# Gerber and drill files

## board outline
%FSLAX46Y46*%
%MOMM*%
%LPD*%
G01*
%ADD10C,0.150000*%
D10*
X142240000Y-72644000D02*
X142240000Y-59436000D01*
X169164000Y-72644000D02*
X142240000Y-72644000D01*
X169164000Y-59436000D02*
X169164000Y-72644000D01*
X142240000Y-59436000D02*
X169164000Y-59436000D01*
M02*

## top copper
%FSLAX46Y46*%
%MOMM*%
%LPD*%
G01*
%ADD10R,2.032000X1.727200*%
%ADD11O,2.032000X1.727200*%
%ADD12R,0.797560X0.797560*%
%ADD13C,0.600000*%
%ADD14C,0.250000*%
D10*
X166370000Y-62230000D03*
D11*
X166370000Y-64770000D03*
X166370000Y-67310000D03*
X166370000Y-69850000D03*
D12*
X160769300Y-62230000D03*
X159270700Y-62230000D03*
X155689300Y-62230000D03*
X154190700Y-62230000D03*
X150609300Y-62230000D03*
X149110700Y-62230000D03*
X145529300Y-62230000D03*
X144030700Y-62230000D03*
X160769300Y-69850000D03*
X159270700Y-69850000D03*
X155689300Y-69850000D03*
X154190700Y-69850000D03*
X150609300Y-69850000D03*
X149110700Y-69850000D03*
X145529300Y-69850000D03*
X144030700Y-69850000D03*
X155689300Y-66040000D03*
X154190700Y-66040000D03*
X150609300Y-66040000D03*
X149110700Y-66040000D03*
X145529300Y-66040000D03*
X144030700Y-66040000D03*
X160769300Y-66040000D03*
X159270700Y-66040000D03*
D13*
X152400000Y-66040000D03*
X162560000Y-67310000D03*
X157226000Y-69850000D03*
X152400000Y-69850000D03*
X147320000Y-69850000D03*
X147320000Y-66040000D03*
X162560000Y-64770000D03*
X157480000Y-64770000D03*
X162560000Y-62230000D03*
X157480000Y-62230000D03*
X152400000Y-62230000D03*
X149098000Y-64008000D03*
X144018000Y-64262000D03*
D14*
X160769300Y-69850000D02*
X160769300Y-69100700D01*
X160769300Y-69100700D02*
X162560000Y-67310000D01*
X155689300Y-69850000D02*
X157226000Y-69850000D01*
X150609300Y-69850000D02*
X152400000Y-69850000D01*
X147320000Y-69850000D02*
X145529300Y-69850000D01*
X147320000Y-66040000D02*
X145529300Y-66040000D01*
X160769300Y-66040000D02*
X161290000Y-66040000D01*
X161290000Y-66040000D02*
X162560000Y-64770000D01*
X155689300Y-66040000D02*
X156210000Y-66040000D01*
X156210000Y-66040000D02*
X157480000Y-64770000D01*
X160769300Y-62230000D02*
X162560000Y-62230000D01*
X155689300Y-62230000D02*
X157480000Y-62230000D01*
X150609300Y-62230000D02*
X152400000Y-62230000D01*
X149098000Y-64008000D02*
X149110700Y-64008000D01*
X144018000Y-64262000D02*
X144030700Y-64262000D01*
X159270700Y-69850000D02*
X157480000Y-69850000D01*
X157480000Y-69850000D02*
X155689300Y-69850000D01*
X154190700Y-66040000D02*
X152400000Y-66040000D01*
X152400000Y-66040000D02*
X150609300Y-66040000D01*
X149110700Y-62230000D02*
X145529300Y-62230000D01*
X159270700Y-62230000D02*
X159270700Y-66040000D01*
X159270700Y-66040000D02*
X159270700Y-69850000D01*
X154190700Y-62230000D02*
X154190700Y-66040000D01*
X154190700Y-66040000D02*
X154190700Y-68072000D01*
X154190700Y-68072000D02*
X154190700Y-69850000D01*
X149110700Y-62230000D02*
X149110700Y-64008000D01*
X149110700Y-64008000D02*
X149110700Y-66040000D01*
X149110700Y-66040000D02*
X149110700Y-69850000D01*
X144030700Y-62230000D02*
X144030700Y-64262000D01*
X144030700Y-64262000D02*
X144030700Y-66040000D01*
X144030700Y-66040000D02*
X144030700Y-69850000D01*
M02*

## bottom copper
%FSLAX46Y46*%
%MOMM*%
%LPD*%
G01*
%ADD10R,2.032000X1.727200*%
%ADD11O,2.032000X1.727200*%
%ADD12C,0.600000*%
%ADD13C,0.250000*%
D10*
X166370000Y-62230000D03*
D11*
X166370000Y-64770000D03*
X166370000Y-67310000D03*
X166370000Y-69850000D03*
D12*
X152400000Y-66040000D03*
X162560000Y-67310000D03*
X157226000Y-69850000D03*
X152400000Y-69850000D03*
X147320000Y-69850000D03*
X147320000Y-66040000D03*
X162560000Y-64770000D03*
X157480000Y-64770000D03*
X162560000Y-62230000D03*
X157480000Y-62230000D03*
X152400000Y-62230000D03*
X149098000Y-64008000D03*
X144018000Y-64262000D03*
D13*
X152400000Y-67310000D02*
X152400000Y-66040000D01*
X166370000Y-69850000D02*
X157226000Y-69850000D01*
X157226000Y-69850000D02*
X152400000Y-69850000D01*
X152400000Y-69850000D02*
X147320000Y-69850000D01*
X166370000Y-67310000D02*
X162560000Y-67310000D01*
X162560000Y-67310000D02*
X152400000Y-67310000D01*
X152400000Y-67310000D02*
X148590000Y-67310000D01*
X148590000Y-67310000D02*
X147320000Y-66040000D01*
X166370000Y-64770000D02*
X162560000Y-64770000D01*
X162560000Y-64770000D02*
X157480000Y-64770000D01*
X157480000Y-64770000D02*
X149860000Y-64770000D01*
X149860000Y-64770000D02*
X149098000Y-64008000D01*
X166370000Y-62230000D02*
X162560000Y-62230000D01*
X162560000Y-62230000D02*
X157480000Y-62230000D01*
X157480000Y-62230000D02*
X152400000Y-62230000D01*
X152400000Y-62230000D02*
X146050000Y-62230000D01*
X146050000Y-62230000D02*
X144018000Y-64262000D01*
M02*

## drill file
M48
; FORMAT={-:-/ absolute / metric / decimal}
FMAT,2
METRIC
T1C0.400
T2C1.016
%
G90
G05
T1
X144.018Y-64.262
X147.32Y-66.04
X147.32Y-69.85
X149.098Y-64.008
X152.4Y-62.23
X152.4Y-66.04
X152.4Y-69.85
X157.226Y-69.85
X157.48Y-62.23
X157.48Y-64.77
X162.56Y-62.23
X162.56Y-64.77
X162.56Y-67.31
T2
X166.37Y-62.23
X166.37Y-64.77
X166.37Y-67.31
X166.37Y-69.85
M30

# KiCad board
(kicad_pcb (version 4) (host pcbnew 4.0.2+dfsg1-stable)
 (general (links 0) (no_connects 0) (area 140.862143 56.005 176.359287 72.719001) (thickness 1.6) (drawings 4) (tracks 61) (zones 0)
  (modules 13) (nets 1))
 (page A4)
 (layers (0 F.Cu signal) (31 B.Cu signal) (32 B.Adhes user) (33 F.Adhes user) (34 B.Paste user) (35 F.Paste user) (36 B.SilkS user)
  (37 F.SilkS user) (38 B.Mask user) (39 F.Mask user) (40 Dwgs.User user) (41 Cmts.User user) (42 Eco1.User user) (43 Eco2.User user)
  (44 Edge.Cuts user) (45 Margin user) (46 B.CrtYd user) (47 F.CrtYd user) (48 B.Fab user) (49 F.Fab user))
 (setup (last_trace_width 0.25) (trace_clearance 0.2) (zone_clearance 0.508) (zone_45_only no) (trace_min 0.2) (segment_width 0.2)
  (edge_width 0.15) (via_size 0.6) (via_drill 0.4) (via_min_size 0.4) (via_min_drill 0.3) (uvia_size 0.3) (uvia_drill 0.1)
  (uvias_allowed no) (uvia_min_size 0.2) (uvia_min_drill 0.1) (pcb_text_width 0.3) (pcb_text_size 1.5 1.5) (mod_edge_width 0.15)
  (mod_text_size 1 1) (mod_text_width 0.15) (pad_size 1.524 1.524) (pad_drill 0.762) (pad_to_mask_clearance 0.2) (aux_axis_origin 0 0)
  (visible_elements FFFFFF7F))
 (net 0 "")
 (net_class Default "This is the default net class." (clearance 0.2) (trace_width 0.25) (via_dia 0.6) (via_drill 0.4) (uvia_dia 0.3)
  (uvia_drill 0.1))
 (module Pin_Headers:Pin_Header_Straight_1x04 (layer F.Cu) (at 166.37 62.23)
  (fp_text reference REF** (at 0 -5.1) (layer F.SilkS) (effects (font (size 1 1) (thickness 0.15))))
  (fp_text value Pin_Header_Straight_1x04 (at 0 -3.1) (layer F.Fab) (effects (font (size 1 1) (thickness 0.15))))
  (pad 1 thru_hole rect (at 0 0) (size 2.032 1.7272) (drill 1.016) (layers *.Cu *.Mask F.SilkS))
  (pad 2 thru_hole oval (at 0 2.54) (size 2.032 1.7272) (drill 1.016) (layers *.Cu *.Mask F.SilkS))
  (pad 3 thru_hole oval (at 0 5.08) (size 2.032 1.7272) (drill 1.016) (layers *.Cu *.Mask F.SilkS))
  (pad 4 thru_hole oval (at 0 7.62) (size 2.032 1.7272) (drill 1.016) (layers *.Cu *.Mask F.SilkS)))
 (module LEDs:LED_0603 (layer F.Cu) (at 160.02 62.23)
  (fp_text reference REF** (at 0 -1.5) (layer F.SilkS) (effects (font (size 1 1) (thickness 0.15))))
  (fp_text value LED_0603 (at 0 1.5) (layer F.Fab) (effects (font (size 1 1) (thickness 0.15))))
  (pad 2 smd rect (at 0.7493 0 180) (size 0.79756 0.79756) (layers F.Cu F.Paste F.Mask))
  (pad 1 smd rect (at -0.7493 0 180) (size 0.79756 0.79756) (layers F.Cu F.Paste F.Mask)))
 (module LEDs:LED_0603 (layer F.Cu) (at 154.94 62.23)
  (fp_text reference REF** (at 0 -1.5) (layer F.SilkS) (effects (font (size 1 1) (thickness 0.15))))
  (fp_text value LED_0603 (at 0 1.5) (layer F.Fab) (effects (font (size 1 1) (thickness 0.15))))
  (pad 2 smd rect (at 0.7493 0 180) (size 0.79756 0.79756) (layers F.Cu F.Paste F.Mask))
  (pad 1 smd rect (at -0.7493 0 180) (size 0.79756 0.79756) (layers F.Cu F.Paste F.Mask)))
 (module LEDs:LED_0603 (layer F.Cu) (at 149.86 62.23)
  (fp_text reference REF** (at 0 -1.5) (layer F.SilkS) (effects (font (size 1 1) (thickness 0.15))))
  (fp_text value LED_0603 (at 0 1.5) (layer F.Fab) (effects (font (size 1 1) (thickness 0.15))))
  (pad 2 smd rect (at 0.7493 0 180) (size 0.79756 0.79756) (layers F.Cu F.Paste F.Mask))
  (pad 1 smd rect (at -0.7493 0 180) (size 0.79756 0.79756) (layers F.Cu F.Paste F.Mask)))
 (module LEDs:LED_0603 (layer F.Cu) (at 144.78 62.23)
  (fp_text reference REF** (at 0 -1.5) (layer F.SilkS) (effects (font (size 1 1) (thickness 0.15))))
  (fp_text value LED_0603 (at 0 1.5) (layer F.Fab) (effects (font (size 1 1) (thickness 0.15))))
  (pad 2 smd rect (at 0.7493 0 180) (size 0.79756 0.79756) (layers F.Cu F.Paste F.Mask))
  (pad 1 smd rect (at -0.7493 0 180) (size 0.79756 0.79756) (layers F.Cu F.Paste F.Mask)))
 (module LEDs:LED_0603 (layer F.Cu) (at 160.02 69.85)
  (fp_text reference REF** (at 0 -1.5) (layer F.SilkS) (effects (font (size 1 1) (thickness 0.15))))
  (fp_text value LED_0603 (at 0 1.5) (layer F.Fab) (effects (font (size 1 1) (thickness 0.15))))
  (pad 2 smd rect (at 0.7493 0 180) (size 0.79756 0.79756) (layers F.Cu F.Paste F.Mask))
  (pad 1 smd rect (at -0.7493 0 180) (size 0.79756 0.79756) (layers F.Cu F.Paste F.Mask)))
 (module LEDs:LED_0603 (layer F.Cu) (at 154.94 69.85)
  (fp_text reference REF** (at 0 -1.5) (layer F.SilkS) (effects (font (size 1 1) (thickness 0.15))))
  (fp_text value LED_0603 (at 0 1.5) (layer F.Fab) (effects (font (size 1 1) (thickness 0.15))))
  (pad 2 smd rect (at 0.7493 0 180) (size 0.79756 0.79756) (layers F.Cu F.Paste F.Mask))
  (pad 1 smd rect (at -0.7493 0 180) (size 0.79756 0.79756) (layers F.Cu F.Paste F.Mask)))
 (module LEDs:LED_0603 (layer F.Cu) (at 149.86 69.85)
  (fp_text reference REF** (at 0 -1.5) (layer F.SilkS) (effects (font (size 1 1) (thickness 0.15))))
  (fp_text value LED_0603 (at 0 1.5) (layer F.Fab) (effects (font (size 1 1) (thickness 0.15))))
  (pad 2 smd rect (at 0.7493 0 180) (size 0.79756 0.79756) (layers F.Cu F.Paste F.Mask))
  (pad 1 smd rect (at -0.7493 0 180) (size 0.79756 0.79756) (layers F.Cu F.Paste F.Mask)))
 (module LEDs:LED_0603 (layer F.Cu) (at 144.78 69.85)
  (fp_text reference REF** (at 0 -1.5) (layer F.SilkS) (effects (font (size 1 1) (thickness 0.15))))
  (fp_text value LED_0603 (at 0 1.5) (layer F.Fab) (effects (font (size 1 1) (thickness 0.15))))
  (pad 2 smd rect (at 0.7493 0 180) (size 0.79756 0.79756) (layers F.Cu F.Paste F.Mask))
  (pad 1 smd rect (at -0.7493 0 180) (size 0.79756 0.79756) (layers F.Cu F.Paste F.Mask)))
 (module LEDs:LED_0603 (layer F.Cu) (at 154.94 66.04)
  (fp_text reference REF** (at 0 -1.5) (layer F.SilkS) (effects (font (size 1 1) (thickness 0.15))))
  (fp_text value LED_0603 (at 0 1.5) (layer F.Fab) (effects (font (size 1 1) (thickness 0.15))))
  (pad 2 smd rect (at 0.7493 0 180) (size 0.79756 0.79756) (layers F.Cu F.Paste F.Mask))
  (pad 1 smd rect (at -0.7493 0 180) (size 0.79756 0.79756) (layers F.Cu F.Paste F.Mask)))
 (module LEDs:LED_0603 (layer F.Cu) (at 149.86 66.04)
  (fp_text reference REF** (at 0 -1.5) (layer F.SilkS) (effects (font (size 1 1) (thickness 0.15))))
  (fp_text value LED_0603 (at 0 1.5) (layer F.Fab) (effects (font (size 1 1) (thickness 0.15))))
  (pad 2 smd rect (at 0.7493 0 180) (size 0.79756 0.79756) (layers F.Cu F.Paste F.Mask))
  (pad 1 smd rect (at -0.7493 0 180) (size 0.79756 0.79756) (layers F.Cu F.Paste F.Mask)))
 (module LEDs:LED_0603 (layer F.Cu) (at 144.78 66.04)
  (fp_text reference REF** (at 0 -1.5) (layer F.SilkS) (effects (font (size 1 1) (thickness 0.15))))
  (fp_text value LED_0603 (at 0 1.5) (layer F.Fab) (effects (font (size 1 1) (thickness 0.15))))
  (pad 2 smd rect (at 0.7493 0 180) (size 0.79756 0.79756) (layers F.Cu F.Paste F.Mask))
  (pad 1 smd rect (at -0.7493 0 180) (size 0.79756 0.79756) (layers F.Cu F.Paste F.Mask)))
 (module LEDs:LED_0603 (layer F.Cu) (at 160.02 66.04)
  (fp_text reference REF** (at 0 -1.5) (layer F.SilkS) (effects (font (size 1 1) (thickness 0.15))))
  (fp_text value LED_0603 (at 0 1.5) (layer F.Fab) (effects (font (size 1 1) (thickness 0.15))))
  (pad 2 smd rect (at 0.7493 0 180) (size 0.79756 0.79756) (layers F.Cu F.Paste F.Mask))
  (pad 1 smd rect (at -0.7493 0 180) (size 0.79756 0.79756) (layers F.Cu F.Paste F.Mask)))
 (gr_line (start 142.24 72.644) (end 142.24 59.436) (angle 90) (layer Edge.Cuts) (width 0.15))
 (gr_line (start 169.164 72.644) (end 142.24 72.644) (angle 90) (layer Edge.Cuts) (width 0.15))
 (gr_line (start 169.164 59.436) (end 169.164 72.644) (angle 90) (layer Edge.Cuts) (width 0.15))
 (gr_line (start 142.24 59.436) (end 169.164 59.436) (angle 90) (layer Edge.Cuts) (width 0.15))
 (segment (start 152.4 67.31) (end 152.4 66.04) (width 0.25) (layer B.Cu) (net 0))
 (via (at 152.4 66.04) (size 0.6) (drill 0.4) (layers F.Cu B.Cu) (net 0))
 (segment (start 160.7693 69.85) (end 160.7693 69.1007) (width 0.25) (layer F.Cu) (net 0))
 (via (at 162.56 67.31) (size 0.6) (drill 0.4) (layers F.Cu B.Cu) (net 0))
 (segment (start 160.7693 69.1007) (end 162.56 67.31) (width 0.25) (layer F.Cu) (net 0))
 (segment (start 155.6893 69.85) (end 157.226 69.85) (width 0.25) (layer F.Cu) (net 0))
 (via (at 157.226 69.85) (size 0.6) (drill 0.4) (layers F.Cu B.Cu) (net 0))
 (segment (start 150.6093 69.85) (end 152.4 69.85) (width 0.25) (layer F.Cu) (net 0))
 (via (at 152.4 69.85) (size 0.6) (drill 0.4) (layers F.Cu B.Cu) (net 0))
 (segment (start 166.37 69.85) (end 157.226 69.85) (width 0.25) (layer B.Cu) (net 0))
 (segment (start 157.226 69.85) (end 152.4 69.85) (width 0.25) (layer B.Cu) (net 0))
 (segment (start 152.4 69.85) (end 147.32 69.85) (width 0.25) (layer B.Cu) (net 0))
 (segment (start 147.32 69.85) (end 145.5293 69.85) (width 0.25) (layer F.Cu) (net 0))
 (via (at 147.32 69.85) (size 0.6) (drill 0.4) (layers F.Cu B.Cu) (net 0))
 (segment (start 166.37 67.31) (end 162.56 67.31) (width 0.25) (layer B.Cu) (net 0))
 (segment (start 162.56 67.31) (end 152.4 67.31) (width 0.25) (layer B.Cu) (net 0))
 (segment (start 152.4 67.31) (end 148.59 67.31) (width 0.25) (layer B.Cu) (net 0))
 (segment (start 147.32 66.04) (end 145.5293 66.04) (width 0.25) (layer F.Cu) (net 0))
 (via (at 147.32 66.04) (size 0.6) (drill 0.4) (layers F.Cu B.Cu) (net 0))
 (segment (start 148.59 67.31) (end 147.32 66.04) (width 0.25) (layer B.Cu) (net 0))
 (segment (start 160.7693 66.04) (end 161.29 66.04) (width 0.25) (layer F.Cu) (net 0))
 (via (at 162.56 64.77) (size 0.6) (drill 0.4) (layers F.Cu B.Cu) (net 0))
 (segment (start 161.29 66.04) (end 162.56 64.77) (width 0.25) (layer F.Cu) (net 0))
 (segment (start 155.6893 66.04) (end 156.21 66.04) (width 0.25) (layer F.Cu) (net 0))
 (via (at 157.48 64.77) (size 0.6) (drill 0.4) (layers F.Cu B.Cu) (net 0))
 (segment (start 156.21 66.04) (end 157.48 64.77) (width 0.25) (layer F.Cu) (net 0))
 (segment (start 160.7693 62.23) (end 162.56 62.23) (width 0.25) (layer F.Cu) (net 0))
 (via (at 162.56 62.23) (size 0.6) (drill 0.4) (layers F.Cu B.Cu) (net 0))
 (segment (start 155.6893 62.23) (end 157.48 62.23) (width 0.25) (layer F.Cu) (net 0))
 (via (at 157.48 62.23) (size 0.6) (drill 0.4) (layers F.Cu B.Cu) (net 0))
 (segment (start 150.6093 62.23) (end 152.4 62.23) (width 0.25) (layer F.Cu) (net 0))
 (via (at 152.4 62.23) (size 0.6) (drill 0.4) (layers F.Cu B.Cu) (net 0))
 (segment (start 166.37 64.77) (end 162.56 64.77) (width 0.25) (layer B.Cu) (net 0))
 (segment (start 162.56 64.77) (end 157.48 64.77) (width 0.25) (layer B.Cu) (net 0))
 (segment (start 157.48 64.77) (end 149.86 64.77) (width 0.25) (layer B.Cu) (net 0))
 (segment (start 149.098 64.008) (end 149.1107 64.008) (width 0.25) (layer F.Cu) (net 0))
 (via (at 149.098 64.008) (size 0.6) (drill 0.4) (layers F.Cu B.Cu) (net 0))
 (segment (start 149.86 64.77) (end 149.098 64.008) (width 0.25) (layer B.Cu) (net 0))
 (segment (start 166.37 62.23) (end 162.56 62.23) (width 0.25) (layer B.Cu) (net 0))
 (segment (start 162.56 62.23) (end 157.48 62.23) (width 0.25) (layer B.Cu) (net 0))
 (segment (start 157.48 62.23) (end 152.4 62.23) (width 0.25) (layer B.Cu) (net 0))
 (segment (start 152.4 62.23) (end 146.05 62.23) (width 0.25) (layer B.Cu) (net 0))
 (segment (start 144.018 64.262) (end 144.0307 64.262) (width 0.25) (layer F.Cu) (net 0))
 (via (at 144.018 64.262) (size 0.6) (drill 0.4) (layers F.Cu B.Cu) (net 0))
 (segment (start 146.05 62.23) (end 144.018 64.262) (width 0.25) (layer B.Cu) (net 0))
 (segment (start 159.2707 69.85) (end 157.48 69.85) (width 0.25) (layer F.Cu) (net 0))
 (segment (start 157.48 69.85) (end 155.6893 69.85) (width 0.25) (layer F.Cu) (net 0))
 (segment (start 154.1907 66.04) (end 152.4 66.04) (width 0.25) (layer F.Cu) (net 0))
 (segment (start 152.4 66.04) (end 150.6093 66.04) (width 0.25) (layer F.Cu) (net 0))
 (segment (start 149.1107 62.23) (end 145.5293 62.23) (width 0.25) (layer F.Cu) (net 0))
 (segment (start 159.2707 62.23) (end 159.2707 66.04) (width 0.25) (layer F.Cu) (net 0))
 (segment (start 159.2707 66.04) (end 159.2707 69.85) (width 0.25) (layer F.Cu) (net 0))
 (segment (start 154.1907 62.23) (end 154.1907 66.04) (width 0.25) (layer F.Cu) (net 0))
 (segment (start 154.1907 66.04) (end 154.1907 68.072) (width 0.25) (layer F.Cu) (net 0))
 (segment (start 154.1907 68.072) (end 154.1907 69.85) (width 0.25) (layer F.Cu) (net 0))
 (segment (start 149.1107 62.23) (end 149.1107 64.008) (width 0.25) (layer F.Cu) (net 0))
 (segment (start 149.1107 64.008) (end 149.1107 66.04) (width 0.25) (layer F.Cu) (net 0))
 (segment (start 149.1107 66.04) (end 149.1107 69.85) (width 0.25) (layer F.Cu) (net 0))
 (segment (start 144.0307 62.23) (end 144.0307 64.262) (width 0.25) (layer F.Cu) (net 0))
 (segment (start 144.0307 64.262) (end 144.0307 66.04) (width 0.25) (layer F.Cu) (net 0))
 (segment (start 144.0307 66.04) (end 144.0307 69.85) (width 0.25) (layer F.Cu) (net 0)))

